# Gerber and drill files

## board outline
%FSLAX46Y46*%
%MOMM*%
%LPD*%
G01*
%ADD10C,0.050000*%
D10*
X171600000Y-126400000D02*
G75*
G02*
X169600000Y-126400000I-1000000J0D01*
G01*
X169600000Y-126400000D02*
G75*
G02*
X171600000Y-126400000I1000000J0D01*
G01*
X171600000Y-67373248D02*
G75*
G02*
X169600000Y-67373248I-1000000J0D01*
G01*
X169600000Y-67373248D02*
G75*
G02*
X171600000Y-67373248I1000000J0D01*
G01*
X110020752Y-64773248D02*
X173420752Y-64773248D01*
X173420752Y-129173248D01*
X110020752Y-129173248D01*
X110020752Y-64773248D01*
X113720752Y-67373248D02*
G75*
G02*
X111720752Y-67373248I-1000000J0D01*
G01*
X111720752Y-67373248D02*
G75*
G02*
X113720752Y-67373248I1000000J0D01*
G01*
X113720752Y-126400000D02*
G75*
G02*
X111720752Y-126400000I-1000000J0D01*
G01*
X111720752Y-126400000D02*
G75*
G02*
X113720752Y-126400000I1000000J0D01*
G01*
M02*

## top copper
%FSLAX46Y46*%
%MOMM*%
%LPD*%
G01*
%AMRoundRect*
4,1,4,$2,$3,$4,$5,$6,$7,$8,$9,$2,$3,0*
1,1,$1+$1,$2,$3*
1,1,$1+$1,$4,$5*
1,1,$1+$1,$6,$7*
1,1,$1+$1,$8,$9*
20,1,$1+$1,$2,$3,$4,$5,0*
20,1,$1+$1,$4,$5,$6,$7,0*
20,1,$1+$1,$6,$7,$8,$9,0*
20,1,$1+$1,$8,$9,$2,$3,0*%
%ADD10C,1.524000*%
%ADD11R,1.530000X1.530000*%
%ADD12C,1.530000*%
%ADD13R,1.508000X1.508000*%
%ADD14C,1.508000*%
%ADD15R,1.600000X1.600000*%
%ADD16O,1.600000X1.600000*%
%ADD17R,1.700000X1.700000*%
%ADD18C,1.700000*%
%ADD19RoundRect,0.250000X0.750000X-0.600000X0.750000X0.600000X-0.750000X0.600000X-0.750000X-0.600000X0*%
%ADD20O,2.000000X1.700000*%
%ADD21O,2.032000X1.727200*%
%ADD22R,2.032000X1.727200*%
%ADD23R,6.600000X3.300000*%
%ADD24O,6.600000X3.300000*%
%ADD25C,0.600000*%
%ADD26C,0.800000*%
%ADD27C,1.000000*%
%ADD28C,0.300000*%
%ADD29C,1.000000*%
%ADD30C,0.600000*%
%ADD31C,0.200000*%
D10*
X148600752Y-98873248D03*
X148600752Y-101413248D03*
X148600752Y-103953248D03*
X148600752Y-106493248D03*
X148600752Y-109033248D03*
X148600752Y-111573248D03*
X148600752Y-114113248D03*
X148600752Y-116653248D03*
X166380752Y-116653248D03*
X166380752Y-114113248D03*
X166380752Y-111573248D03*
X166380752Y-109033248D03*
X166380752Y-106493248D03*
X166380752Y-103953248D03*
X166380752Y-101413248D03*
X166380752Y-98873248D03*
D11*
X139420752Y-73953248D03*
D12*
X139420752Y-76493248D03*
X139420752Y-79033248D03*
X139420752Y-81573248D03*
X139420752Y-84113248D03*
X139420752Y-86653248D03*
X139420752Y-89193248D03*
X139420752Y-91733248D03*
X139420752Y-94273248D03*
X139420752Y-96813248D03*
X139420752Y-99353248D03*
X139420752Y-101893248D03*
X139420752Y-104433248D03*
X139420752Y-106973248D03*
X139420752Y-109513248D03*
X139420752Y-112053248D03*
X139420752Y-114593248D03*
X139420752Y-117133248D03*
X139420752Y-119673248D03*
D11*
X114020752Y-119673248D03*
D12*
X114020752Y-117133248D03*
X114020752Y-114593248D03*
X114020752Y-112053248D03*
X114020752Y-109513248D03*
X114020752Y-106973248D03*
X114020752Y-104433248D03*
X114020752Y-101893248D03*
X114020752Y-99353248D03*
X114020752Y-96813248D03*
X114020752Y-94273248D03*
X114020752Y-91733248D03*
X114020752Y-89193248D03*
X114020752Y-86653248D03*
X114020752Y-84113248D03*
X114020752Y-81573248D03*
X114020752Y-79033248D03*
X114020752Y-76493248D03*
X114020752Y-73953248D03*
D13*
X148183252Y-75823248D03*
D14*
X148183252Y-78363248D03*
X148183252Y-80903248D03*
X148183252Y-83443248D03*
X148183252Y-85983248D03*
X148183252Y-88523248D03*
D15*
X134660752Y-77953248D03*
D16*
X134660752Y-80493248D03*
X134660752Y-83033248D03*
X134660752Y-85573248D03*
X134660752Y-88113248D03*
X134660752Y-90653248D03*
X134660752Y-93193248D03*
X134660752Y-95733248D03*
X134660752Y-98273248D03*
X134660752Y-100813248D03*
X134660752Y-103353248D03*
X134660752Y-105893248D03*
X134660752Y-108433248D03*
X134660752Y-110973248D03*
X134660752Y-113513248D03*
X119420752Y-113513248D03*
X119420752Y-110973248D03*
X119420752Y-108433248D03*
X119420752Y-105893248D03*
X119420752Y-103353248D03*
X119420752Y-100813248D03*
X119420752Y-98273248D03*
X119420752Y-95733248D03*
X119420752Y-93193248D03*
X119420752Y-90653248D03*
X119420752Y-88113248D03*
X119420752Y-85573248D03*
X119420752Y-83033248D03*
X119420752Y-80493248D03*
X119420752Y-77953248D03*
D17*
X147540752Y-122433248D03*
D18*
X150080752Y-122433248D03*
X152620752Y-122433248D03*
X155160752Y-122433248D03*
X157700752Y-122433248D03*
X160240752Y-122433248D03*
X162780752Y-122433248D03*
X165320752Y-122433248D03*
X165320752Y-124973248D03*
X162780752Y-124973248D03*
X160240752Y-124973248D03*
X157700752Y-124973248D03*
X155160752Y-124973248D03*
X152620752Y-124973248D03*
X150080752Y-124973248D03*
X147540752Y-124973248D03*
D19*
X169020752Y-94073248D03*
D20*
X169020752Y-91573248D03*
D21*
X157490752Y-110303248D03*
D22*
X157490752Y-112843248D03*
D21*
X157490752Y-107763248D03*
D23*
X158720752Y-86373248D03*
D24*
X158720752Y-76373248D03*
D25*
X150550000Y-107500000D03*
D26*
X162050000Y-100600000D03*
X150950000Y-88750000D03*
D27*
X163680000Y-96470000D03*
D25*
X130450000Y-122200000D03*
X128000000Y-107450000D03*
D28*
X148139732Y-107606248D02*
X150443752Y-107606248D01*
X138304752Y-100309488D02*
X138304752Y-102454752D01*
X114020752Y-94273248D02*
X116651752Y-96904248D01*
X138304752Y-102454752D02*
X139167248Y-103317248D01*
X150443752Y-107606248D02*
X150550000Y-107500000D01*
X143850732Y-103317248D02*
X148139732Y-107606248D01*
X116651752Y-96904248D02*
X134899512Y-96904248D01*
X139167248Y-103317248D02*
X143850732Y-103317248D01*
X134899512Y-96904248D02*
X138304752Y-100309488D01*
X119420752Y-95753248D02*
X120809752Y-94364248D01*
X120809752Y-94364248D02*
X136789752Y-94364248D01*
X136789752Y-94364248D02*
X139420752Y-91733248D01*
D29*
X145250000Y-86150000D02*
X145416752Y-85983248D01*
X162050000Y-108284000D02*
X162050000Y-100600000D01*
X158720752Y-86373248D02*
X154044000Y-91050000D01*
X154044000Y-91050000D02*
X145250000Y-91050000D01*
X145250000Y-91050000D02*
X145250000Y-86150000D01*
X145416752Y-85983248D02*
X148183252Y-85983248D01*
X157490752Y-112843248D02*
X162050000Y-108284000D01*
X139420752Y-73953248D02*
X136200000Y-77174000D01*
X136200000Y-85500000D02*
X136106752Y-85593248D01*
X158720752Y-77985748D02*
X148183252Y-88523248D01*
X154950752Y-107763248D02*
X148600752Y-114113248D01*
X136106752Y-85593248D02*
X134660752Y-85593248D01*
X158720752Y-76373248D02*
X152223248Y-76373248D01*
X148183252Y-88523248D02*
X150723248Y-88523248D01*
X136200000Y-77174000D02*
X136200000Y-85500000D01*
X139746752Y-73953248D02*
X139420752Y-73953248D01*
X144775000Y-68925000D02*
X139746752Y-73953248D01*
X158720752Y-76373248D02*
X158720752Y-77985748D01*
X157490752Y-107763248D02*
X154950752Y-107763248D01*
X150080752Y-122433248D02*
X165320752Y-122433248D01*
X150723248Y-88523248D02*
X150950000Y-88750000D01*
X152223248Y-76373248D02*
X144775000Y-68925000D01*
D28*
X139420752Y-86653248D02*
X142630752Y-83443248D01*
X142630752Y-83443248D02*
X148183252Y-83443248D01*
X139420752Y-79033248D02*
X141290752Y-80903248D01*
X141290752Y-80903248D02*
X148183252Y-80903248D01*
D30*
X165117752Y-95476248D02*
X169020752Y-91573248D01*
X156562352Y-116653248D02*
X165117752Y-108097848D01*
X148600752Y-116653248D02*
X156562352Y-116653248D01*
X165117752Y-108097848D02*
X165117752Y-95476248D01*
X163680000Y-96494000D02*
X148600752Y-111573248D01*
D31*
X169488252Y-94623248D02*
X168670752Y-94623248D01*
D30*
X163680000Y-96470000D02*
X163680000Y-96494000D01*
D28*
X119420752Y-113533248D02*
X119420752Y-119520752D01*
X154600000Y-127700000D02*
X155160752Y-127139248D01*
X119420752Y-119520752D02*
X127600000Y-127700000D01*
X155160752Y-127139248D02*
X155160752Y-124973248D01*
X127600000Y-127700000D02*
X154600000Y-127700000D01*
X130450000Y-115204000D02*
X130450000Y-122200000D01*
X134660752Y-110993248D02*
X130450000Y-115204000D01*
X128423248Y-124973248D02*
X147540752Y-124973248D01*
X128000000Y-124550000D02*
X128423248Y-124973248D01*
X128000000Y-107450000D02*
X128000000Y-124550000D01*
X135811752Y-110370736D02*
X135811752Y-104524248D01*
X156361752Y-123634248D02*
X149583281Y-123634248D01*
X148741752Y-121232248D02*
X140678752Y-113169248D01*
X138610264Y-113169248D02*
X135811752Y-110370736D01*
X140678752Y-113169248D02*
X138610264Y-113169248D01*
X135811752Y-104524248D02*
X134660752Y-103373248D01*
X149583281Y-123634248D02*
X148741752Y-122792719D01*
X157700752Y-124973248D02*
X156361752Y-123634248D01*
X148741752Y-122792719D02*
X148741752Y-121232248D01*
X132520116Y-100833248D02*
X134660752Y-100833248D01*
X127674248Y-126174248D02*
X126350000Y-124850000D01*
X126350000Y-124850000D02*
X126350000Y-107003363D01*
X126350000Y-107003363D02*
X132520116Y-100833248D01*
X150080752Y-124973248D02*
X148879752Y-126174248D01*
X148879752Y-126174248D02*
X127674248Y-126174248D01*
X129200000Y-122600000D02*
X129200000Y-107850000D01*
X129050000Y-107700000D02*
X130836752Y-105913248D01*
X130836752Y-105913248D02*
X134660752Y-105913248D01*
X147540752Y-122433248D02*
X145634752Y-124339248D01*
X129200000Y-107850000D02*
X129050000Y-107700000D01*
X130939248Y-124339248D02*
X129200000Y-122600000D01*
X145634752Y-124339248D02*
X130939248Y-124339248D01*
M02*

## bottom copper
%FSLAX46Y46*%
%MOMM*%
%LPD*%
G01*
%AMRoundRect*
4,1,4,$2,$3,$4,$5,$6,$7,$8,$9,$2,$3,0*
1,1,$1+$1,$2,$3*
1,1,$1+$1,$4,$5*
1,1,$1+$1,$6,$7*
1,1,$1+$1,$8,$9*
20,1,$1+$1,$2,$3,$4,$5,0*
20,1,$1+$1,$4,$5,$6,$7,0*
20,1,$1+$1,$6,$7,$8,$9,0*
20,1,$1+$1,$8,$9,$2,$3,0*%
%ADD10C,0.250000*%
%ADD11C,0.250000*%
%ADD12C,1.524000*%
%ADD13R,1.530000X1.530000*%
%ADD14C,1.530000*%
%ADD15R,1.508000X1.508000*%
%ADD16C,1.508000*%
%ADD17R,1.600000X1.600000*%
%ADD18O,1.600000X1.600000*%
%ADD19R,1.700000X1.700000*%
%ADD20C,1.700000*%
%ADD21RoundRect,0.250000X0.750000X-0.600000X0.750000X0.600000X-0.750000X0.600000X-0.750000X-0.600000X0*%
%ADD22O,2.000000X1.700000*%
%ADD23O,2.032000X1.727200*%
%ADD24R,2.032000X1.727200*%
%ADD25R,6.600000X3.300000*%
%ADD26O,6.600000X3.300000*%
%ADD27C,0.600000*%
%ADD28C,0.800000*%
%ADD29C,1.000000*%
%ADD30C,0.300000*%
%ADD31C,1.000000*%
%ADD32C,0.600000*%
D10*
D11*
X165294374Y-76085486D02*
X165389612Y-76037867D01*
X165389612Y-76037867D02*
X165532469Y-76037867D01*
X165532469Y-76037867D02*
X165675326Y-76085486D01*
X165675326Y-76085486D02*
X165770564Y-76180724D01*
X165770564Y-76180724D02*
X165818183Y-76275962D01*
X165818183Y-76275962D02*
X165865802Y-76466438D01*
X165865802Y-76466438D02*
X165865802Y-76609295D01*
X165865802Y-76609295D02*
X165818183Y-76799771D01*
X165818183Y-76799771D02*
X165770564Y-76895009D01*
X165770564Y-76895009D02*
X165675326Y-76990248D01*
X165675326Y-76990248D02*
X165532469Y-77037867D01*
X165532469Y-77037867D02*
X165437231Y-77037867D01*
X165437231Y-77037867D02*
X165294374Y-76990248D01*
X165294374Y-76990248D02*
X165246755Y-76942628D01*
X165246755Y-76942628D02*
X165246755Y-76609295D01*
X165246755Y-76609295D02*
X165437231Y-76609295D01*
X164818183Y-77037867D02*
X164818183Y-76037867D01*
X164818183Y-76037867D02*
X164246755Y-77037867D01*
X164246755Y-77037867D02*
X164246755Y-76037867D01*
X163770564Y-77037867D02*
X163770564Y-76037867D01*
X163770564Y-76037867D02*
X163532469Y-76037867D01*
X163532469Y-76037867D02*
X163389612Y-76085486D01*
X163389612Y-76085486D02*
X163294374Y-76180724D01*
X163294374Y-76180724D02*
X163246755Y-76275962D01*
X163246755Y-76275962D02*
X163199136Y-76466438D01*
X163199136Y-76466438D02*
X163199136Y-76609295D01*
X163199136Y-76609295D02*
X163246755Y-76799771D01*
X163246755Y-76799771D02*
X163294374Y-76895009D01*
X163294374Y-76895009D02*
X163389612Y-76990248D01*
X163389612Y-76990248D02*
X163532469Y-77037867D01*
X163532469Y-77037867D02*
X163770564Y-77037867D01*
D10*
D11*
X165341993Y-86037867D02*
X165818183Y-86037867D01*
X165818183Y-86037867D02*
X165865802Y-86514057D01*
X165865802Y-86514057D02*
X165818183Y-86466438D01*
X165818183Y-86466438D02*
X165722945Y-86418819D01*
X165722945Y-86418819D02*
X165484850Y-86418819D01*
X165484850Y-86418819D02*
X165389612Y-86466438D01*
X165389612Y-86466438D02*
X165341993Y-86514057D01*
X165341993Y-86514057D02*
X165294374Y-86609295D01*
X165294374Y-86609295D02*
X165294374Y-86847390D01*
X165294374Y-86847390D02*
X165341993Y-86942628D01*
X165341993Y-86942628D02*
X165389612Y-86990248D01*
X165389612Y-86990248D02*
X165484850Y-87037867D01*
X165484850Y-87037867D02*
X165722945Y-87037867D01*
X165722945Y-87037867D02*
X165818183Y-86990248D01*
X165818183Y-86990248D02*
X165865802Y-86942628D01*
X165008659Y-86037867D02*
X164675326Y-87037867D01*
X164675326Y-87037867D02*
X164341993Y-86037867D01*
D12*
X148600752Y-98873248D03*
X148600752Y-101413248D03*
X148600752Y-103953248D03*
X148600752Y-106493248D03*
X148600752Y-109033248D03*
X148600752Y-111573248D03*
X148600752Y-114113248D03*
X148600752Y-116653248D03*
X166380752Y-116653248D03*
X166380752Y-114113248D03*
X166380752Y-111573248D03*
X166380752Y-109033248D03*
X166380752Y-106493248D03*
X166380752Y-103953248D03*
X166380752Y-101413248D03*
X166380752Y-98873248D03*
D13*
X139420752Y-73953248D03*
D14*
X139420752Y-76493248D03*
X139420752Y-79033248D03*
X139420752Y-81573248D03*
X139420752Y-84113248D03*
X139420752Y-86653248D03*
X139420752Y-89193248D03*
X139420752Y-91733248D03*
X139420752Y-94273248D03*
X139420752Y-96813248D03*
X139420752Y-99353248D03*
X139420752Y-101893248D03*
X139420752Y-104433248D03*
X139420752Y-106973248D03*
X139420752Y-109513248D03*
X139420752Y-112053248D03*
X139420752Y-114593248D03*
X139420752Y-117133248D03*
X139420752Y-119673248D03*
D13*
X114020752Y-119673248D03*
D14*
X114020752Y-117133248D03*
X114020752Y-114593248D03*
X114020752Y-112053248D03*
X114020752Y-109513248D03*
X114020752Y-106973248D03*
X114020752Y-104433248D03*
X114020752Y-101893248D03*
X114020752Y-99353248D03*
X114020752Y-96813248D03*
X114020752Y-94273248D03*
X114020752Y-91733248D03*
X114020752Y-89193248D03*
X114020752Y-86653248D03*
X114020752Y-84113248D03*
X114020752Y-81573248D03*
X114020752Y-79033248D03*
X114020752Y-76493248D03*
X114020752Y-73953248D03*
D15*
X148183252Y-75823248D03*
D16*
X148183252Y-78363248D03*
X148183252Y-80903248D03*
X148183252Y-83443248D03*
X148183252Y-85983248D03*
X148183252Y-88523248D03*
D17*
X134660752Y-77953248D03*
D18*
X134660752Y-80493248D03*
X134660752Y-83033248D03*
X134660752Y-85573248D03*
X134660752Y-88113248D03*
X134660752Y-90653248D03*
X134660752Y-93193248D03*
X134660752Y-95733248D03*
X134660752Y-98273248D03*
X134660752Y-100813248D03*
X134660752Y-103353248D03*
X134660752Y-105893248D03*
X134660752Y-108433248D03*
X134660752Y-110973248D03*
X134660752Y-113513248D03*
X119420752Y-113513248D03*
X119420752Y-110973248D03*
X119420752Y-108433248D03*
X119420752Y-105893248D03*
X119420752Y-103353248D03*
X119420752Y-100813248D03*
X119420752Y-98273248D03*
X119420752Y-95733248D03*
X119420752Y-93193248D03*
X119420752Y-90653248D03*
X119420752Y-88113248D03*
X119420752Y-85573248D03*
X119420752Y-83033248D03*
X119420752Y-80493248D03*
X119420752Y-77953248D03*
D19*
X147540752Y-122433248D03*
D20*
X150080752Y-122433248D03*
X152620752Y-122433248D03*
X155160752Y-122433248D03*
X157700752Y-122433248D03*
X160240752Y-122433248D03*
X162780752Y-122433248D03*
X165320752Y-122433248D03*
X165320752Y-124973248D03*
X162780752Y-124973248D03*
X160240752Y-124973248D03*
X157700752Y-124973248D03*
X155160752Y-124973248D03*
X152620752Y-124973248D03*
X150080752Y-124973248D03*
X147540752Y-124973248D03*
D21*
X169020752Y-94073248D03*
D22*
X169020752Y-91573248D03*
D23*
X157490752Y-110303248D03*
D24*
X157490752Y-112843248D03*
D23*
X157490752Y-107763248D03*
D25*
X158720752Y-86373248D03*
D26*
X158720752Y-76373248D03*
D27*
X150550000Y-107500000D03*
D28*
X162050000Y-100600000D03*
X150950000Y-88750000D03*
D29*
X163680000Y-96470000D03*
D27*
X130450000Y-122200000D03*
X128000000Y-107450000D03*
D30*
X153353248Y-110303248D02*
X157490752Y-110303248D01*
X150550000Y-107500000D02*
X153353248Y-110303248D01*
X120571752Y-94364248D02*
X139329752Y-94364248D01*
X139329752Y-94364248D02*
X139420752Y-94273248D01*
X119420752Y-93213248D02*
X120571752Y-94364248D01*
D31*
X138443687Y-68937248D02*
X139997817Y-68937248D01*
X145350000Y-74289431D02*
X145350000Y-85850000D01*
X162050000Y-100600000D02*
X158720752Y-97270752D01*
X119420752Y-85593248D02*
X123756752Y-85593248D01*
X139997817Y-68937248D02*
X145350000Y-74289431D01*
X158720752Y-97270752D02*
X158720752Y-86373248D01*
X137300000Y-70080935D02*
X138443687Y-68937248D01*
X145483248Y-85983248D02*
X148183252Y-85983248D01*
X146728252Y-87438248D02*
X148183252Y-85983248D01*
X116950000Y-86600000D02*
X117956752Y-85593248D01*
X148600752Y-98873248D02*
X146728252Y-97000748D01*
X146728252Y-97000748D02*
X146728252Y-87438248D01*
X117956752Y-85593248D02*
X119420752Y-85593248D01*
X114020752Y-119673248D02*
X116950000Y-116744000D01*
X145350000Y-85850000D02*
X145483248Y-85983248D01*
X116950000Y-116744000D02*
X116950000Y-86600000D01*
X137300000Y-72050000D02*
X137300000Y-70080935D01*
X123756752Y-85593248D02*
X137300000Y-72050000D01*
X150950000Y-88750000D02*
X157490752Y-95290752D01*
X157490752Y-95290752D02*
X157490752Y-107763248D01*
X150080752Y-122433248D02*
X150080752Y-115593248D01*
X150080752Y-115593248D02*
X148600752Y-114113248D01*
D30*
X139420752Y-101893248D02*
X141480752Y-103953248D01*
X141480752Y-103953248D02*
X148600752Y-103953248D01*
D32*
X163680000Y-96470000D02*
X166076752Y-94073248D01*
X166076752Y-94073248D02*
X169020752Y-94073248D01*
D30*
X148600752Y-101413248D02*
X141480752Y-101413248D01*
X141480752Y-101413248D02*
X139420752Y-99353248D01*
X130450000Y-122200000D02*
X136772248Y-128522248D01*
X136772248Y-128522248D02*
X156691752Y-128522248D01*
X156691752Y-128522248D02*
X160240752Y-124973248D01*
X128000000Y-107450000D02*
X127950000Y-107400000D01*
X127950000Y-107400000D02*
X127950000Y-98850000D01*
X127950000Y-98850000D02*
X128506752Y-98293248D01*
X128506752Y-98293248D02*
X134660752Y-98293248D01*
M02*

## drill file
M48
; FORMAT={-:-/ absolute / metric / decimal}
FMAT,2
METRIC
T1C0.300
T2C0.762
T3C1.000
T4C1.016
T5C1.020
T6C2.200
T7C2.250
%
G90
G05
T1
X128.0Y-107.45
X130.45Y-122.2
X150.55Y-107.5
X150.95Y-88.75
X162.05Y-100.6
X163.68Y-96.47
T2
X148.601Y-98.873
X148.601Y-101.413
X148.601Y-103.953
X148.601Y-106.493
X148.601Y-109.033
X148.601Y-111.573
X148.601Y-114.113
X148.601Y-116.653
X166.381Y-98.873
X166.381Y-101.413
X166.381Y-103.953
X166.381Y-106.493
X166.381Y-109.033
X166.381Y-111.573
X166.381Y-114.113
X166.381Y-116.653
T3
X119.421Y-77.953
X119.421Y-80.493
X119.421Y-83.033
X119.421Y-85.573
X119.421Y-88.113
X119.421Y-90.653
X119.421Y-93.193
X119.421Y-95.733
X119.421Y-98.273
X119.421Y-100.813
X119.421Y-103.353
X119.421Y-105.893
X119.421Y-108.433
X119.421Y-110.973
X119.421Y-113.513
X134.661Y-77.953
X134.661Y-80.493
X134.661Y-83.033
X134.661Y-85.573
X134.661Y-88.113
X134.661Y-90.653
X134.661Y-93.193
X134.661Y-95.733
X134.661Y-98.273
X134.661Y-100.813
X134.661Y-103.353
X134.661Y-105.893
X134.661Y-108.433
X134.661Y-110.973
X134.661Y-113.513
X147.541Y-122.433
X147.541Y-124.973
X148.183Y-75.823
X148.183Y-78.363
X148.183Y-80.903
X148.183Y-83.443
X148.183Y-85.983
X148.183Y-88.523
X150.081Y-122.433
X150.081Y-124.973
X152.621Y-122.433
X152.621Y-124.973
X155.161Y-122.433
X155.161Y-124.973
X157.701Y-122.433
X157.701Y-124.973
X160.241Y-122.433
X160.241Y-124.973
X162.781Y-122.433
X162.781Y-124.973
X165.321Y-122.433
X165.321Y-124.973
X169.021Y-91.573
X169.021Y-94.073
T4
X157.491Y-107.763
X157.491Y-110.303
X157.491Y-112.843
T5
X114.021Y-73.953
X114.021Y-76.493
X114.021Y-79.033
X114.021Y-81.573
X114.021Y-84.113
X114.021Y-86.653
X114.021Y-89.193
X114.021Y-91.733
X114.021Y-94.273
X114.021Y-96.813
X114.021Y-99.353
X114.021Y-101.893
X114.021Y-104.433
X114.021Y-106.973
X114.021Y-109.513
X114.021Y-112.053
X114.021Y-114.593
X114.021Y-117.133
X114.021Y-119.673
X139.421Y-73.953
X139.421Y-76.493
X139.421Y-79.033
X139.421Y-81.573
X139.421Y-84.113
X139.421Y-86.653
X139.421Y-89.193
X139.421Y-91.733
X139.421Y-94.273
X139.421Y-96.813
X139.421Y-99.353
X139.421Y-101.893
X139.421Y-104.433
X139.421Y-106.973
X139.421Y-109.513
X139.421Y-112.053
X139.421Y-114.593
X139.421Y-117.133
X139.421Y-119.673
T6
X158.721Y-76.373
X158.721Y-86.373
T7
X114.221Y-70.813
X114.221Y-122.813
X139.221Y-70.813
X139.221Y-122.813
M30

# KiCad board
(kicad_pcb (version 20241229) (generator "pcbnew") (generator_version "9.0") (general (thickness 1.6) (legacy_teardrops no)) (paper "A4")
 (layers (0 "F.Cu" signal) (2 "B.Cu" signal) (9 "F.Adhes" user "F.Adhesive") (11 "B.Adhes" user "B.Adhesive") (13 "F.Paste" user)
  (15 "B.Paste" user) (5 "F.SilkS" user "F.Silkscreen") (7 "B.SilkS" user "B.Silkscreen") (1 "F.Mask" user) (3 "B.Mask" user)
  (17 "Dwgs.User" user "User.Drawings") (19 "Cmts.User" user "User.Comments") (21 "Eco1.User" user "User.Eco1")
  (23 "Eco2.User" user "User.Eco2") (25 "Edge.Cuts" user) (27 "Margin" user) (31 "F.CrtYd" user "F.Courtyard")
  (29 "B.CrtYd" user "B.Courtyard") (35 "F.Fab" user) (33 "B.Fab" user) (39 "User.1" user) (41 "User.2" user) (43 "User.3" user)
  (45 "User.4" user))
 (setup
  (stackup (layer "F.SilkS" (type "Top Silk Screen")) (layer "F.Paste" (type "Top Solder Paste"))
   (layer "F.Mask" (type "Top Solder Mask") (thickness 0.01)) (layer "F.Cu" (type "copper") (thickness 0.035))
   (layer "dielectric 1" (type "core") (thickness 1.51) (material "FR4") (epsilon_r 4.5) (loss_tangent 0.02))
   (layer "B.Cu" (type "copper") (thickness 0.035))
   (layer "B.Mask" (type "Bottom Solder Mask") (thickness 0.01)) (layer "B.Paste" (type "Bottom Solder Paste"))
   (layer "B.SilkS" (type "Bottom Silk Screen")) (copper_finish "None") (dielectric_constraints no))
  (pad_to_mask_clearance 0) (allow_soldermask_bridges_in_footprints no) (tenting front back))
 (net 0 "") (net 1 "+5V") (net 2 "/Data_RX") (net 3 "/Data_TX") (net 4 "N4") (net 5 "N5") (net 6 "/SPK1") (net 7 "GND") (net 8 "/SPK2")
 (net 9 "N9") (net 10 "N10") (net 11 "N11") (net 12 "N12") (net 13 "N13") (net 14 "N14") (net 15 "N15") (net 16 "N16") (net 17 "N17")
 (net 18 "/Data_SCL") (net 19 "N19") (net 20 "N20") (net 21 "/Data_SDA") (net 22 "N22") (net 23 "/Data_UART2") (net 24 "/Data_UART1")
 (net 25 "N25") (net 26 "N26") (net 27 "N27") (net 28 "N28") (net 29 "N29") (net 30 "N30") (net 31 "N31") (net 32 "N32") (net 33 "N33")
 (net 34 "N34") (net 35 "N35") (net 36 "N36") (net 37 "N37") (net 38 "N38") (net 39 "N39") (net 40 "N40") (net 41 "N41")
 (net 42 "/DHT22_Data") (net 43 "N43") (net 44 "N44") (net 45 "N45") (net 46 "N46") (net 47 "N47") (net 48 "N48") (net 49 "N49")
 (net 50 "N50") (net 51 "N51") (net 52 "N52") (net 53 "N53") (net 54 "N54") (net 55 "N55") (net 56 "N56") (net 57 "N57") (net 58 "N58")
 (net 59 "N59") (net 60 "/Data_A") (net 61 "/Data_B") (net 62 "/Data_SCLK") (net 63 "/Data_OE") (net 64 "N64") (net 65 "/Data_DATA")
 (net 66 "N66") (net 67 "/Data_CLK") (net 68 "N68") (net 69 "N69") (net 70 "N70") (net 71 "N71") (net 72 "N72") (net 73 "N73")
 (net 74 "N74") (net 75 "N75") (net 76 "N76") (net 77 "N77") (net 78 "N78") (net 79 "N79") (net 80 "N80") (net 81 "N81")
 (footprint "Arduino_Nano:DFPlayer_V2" (layer "F.Cu") (at 156.220752 98.873248)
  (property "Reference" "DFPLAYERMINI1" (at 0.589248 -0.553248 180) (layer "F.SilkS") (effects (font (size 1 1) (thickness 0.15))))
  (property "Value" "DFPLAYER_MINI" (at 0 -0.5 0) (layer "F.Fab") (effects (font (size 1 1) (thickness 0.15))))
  (pad "1" thru_hole circle (at -7.62 0) (size 1.524 1.524) (drill 0.762) (layers "*.Cu" "*.Mask") (remove_unused_layers no) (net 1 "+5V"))
  (pad "2" thru_hole circle (at -7.62 2.54) (size 1.524 1.524) (drill 0.762) (layers "*.Cu" "*.Mask") (remove_unused_layers no)
   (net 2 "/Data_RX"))
  (pad "3" thru_hole circle (at -7.62 5.08) (size 1.524 1.524) (drill 0.762) (layers "*.Cu" "*.Mask") (remove_unused_layers no)
   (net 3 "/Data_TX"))
  (pad "4" thru_hole circle (at -7.62 7.62) (size 1.524 1.524) (drill 0.762) (layers "*.Cu" "*.Mask") (remove_unused_layers no) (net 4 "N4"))
  (pad "5" thru_hole circle (at -7.62 10.16) (size 1.524 1.524) (drill 0.762) (layers "*.Cu" "*.Mask") (remove_unused_layers no)
   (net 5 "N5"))
  (pad "6" thru_hole circle (at -7.62 12.7) (size 1.524 1.524) (drill 0.762) (layers "*.Cu" "*.Mask") (remove_unused_layers no)
   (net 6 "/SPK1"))
  (pad "7" thru_hole circle (at -7.62 15.24) (size 1.524 1.524) (drill 0.762) (layers "*.Cu" "*.Mask") (remove_unused_layers no)
   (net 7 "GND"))
  (pad "8" thru_hole circle (at -7.62 17.78) (size 1.524 1.524) (drill 0.762) (layers "*.Cu" "*.Mask") (remove_unused_layers no)
   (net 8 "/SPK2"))
  (pad "9" thru_hole circle (at 10.16 17.78) (size 1.524 1.524) (drill 0.762) (layers "*.Cu" "*.Mask") (remove_unused_layers no)
   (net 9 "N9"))
  (pad "10" thru_hole circle (at 10.16 15.24) (size 1.524 1.524) (drill 0.762) (layers "*.Cu" "*.Mask") (remove_unused_layers no)
   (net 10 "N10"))
  (pad "11" thru_hole circle (at 10.16 12.7) (size 1.524 1.524) (drill 0.762) (layers "*.Cu" "*.Mask") (remove_unused_layers no)
   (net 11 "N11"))
  (pad "12" thru_hole circle (at 10.16 10.16) (size 1.524 1.524) (drill 0.762) (layers "*.Cu" "*.Mask") (remove_unused_layers no)
   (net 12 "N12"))
  (pad "13" thru_hole circle (at 10.16 7.62) (size 1.524 1.524) (drill 0.762) (layers "*.Cu" "*.Mask") (remove_unused_layers no)
   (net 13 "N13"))
  (pad "14" thru_hole circle (at 10.16 5.08) (size 1.524 1.524) (drill 0.762) (layers "*.Cu" "*.Mask") (remove_unused_layers no)
   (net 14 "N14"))
  (pad "15" thru_hole circle (at 10.16 2.54) (size 1.524 1.524) (drill 0.762) (layers "*.Cu" "*.Mask") (remove_unused_layers no)
   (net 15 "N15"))
  (pad "16" thru_hole circle (at 10.16 0) (size 1.524 1.524) (drill 0.762) (layers "*.Cu" "*.Mask") (remove_unused_layers no) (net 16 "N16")))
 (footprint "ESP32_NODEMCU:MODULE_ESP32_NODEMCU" (layer "F.Cu") (at 126.720752 96.813248)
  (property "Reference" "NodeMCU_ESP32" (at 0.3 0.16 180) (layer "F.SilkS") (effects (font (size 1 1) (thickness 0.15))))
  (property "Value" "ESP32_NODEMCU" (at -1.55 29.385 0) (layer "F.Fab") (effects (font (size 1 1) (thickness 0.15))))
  (pad "" np_thru_hole circle (at -12.5 -26) (size 2.25 2.25) (drill 2.25) (layers "*.Cu" "*.Mask"))
  (pad "" np_thru_hole circle (at -12.5 26) (size 2.25 2.25) (drill 2.25) (layers "*.Cu" "*.Mask"))
  (pad "" np_thru_hole circle (at 12.5 -26) (size 2.25 2.25) (drill 2.25) (layers "*.Cu" "*.Mask"))
  (pad "" np_thru_hole circle (at 12.5 26) (size 2.25 2.25) (drill 2.25) (layers "*.Cu" "*.Mask"))
  (pad "J4_1" thru_hole rect (at 12.7 -22.86) (size 1.53 1.53) (drill 1.02) (layers "*.Cu" "*.Mask") (remove_unused_layers no) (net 7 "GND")
   (solder_mask_margin 0.102))
  (pad "J4_2" thru_hole circle (at 12.7 -20.32) (size 1.53 1.53) (drill 1.02) (layers "*.Cu" "*.Mask") (remove_unused_layers no)
   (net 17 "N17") (solder_mask_margin 0.102))
  (pad "J4_3" thru_hole circle (at 12.7 -17.78) (size 1.53 1.53) (drill 1.02) (layers "*.Cu" "*.Mask") (remove_unused_layers no)
   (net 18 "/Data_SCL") (solder_mask_margin 0.102))
  (pad "J4_4" thru_hole circle (at 12.7 -15.24) (size 1.53 1.53) (drill 1.02) (layers "*.Cu" "*.Mask") (remove_unused_layers no)
   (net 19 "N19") (solder_mask_margin 0.102))
  (pad "J4_5" thru_hole circle (at 12.7 -12.7) (size 1.53 1.53) (drill 1.02) (layers "*.Cu" "*.Mask") (remove_unused_layers no)
   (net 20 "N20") (solder_mask_margin 0.102))
  (pad "J4_6" thru_hole circle (at 12.7 -10.16) (size 1.53 1.53) (drill 1.02) (layers "*.Cu" "*.Mask") (remove_unused_layers no)
   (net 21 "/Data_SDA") (solder_mask_margin 0.102))
  (pad "J4_7" thru_hole circle (at 12.7 -7.62) (size 1.53 1.53) (drill 1.02) (layers "*.Cu" "*.Mask") (remove_unused_layers no)
   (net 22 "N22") (solder_mask_margin 0.102))
  (pad "J4_8" thru_hole circle (at 12.7 -5.08) (size 1.53 1.53) (drill 1.02) (layers "*.Cu" "*.Mask") (remove_unused_layers no)
   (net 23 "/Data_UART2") (solder_mask_margin 0.102))
  (pad "J4_9" thru_hole circle (at 12.7 -2.54) (size 1.53 1.53) (drill 1.02) (layers "*.Cu" "*.Mask") (remove_unused_layers no)
   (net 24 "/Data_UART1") (solder_mask_margin 0.102))
  (pad "J4_10" thru_hole circle (at 12.7 0) (size 1.53 1.53) (drill 1.02) (layers "*.Cu" "*.Mask") (remove_unused_layers no) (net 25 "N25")
   (solder_mask_margin 0.102))
  (pad "J4_11" thru_hole circle (at 12.7 2.54) (size 1.53 1.53) (drill 1.02) (layers "*.Cu" "*.Mask") (remove_unused_layers no)
   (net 2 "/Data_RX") (solder_mask_margin 0.102))
  (pad "J4_12" thru_hole circle (at 12.7 5.08) (size 1.53 1.53) (drill 1.02) (layers "*.Cu" "*.Mask") (remove_unused_layers no)
   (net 3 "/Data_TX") (solder_mask_margin 0.102))
  (pad "J4_13" thru_hole circle (at 12.7 7.62) (size 1.53 1.53) (drill 1.02) (layers "*.Cu" "*.Mask") (remove_unused_layers no)
   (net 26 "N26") (solder_mask_margin 0.102))
  (pad "J4_14" thru_hole circle (at 12.7 10.16) (size 1.53 1.53) (drill 1.02) (layers "*.Cu" "*.Mask") (remove_unused_layers no)
   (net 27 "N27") (solder_mask_margin 0.102))
  (pad "J4_15" thru_hole circle (at 12.7 12.7) (size 1.53 1.53) (drill 1.02) (layers "*.Cu" "*.Mask") (remove_unused_layers no)
   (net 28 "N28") (solder_mask_margin 0.102))
  (pad "J4_16" thru_hole circle (at 12.7 15.24) (size 1.53 1.53) (drill 1.02) (layers "*.Cu" "*.Mask") (remove_unused_layers no)
   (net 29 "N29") (solder_mask_margin 0.102))
  (pad "J4_17" thru_hole circle (at 12.7 17.78) (size 1.53 1.53) (drill 1.02) (layers "*.Cu" "*.Mask") (remove_unused_layers no)
   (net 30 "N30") (solder_mask_margin 0.102))
  (pad "J4_18" thru_hole circle (at 12.7 20.32) (size 1.53 1.53) (drill 1.02) (layers "*.Cu" "*.Mask") (remove_unused_layers no)
   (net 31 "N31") (solder_mask_margin 0.102))
  (pad "J4_19" thru_hole circle (at 12.7 22.86) (size 1.53 1.53) (drill 1.02) (layers "*.Cu" "*.Mask") (remove_unused_layers no)
   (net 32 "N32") (solder_mask_margin 0.102))
  (pad "J5_1" thru_hole rect (at -12.7 22.86) (size 1.53 1.53) (drill 1.02) (layers "*.Cu" "*.Mask") (remove_unused_layers no) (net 1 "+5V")
   (solder_mask_margin 0.102))
  (pad "J5_2" thru_hole circle (at -12.7 20.32) (size 1.53 1.53) (drill 1.02) (layers "*.Cu" "*.Mask") (remove_unused_layers no)
   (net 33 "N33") (solder_mask_margin 0.102))
  (pad "J5_3" thru_hole circle (at -12.7 17.78) (size 1.53 1.53) (drill 1.02) (layers "*.Cu" "*.Mask") (remove_unused_layers no)
   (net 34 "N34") (solder_mask_margin 0.102))
  (pad "J5_4" thru_hole circle (at -12.7 15.24) (size 1.53 1.53) (drill 1.02) (layers "*.Cu" "*.Mask") (remove_unused_layers no)
   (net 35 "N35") (solder_mask_margin 0.102))
  (pad "J5_5" thru_hole circle (at -12.7 12.7) (size 1.53 1.53) (drill 1.02) (layers "*.Cu" "*.Mask") (remove_unused_layers no)
   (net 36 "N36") (solder_mask_margin 0.102))
  (pad "J5_6" thru_hole circle (at -12.7 10.16) (size 1.53 1.53) (drill 1.02) (layers "*.Cu" "*.Mask") (remove_unused_layers no)
   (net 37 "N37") (solder_mask_margin 0.102))
  (pad "J5_7" thru_hole circle (at -12.7 7.62) (size 1.53 1.53) (drill 1.02) (layers "*.Cu" "*.Mask") (remove_unused_layers no)
   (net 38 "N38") (solder_mask_margin 0.102))
  (pad "J5_8" thru_hole circle (at -12.7 5.08) (size 1.53 1.53) (drill 1.02) (layers "*.Cu" "*.Mask") (remove_unused_layers no)
   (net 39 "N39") (solder_mask_margin 0.102))
  (pad "J5_9" thru_hole circle (at -12.7 2.54) (size 1.53 1.53) (drill 1.02) (layers "*.Cu" "*.Mask") (remove_unused_layers no)
   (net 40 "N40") (solder_mask_margin 0.102))
  (pad "J5_10" thru_hole circle (at -12.7 0) (size 1.53 1.53) (drill 1.02) (layers "*.Cu" "*.Mask") (remove_unused_layers no) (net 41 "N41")
   (solder_mask_margin 0.102))
  (pad "J5_11" thru_hole circle (at -12.7 -2.54) (size 1.53 1.53) (drill 1.02) (layers "*.Cu" "*.Mask") (remove_unused_layers no)
   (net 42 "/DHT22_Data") (solder_mask_margin 0.102))
  (pad "J5_12" thru_hole circle (at -12.7 -5.08) (size 1.53 1.53) (drill 1.02) (layers "*.Cu" "*.Mask") (remove_unused_layers no)
   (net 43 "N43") (solder_mask_margin 0.102))
  (pad "J5_13" thru_hole circle (at -12.7 -7.62) (size 1.53 1.53) (drill 1.02) (layers "*.Cu" "*.Mask") (remove_unused_layers no)
   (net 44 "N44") (solder_mask_margin 0.102))
  (pad "J5_14" thru_hole circle (at -12.7 -10.16) (size 1.53 1.53) (drill 1.02) (layers "*.Cu" "*.Mask") (remove_unused_layers no)
   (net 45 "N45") (solder_mask_margin 0.102))
  (pad "J5_15" thru_hole circle (at -12.7 -12.7) (size 1.53 1.53) (drill 1.02) (layers "*.Cu" "*.Mask") (remove_unused_layers no)
   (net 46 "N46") (solder_mask_margin 0.102))
  (pad "J5_16" thru_hole circle (at -12.7 -15.24) (size 1.53 1.53) (drill 1.02) (layers "*.Cu" "*.Mask") (remove_unused_layers no)
   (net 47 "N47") (solder_mask_margin 0.102))
  (pad "J5_17" thru_hole circle (at -12.7 -17.78) (size 1.53 1.53) (drill 1.02) (layers "*.Cu" "*.Mask") (remove_unused_layers no)
   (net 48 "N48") (solder_mask_margin 0.102))
  (pad "J5_18" thru_hole circle (at -12.7 -20.32) (size 1.53 1.53) (drill 1.02) (layers "*.Cu" "*.Mask") (remove_unused_layers no)
   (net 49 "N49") (solder_mask_margin 0.102))
  (pad "J5_19" thru_hole circle (at -12.7 -22.86) (size 1.53 1.53) (drill 1.02) (layers "*.Cu" "*.Mask") (remove_unused_layers no)
   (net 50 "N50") (solder_mask_margin 0.102)))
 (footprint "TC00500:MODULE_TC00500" (layer "F.Cu") (at 148.183252 82.173248)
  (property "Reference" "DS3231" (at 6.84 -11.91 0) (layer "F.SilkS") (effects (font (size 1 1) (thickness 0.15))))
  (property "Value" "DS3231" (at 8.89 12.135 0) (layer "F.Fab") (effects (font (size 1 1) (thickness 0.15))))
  (pad "1" thru_hole rect (at 0 -6.35) (size 1.508 1.508) (drill 1) (layers "*.Cu" "*.Mask") (remove_unused_layers no) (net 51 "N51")
   (solder_mask_margin 0.102))
  (pad "2" thru_hole circle (at 0 -3.81) (size 1.508 1.508) (drill 1) (layers "*.Cu" "*.Mask") (remove_unused_layers no) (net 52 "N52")
   (solder_mask_margin 0.102))
  (pad "3" thru_hole circle (at 0 -1.27) (size 1.508 1.508) (drill 1) (layers "*.Cu" "*.Mask") (remove_unused_layers no)
   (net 18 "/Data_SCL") (solder_mask_margin 0.102))
  (pad "4" thru_hole circle (at 0 1.27) (size 1.508 1.508) (drill 1) (layers "*.Cu" "*.Mask") (remove_unused_layers no) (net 21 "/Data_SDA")
   (solder_mask_margin 0.102))
  (pad "5" thru_hole circle (at 0 3.81) (size 1.508 1.508) (drill 1) (layers "*.Cu" "*.Mask") (remove_unused_layers no) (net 1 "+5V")
   (solder_mask_margin 0.102))
  (pad "6" thru_hole circle (at 0 6.35) (size 1.508 1.508) (drill 1) (layers "*.Cu" "*.Mask") (remove_unused_layers no) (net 7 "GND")
   (solder_mask_margin 0.102)))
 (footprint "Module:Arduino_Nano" (layer "B.Cu") (at 134.660752 77.953248 180)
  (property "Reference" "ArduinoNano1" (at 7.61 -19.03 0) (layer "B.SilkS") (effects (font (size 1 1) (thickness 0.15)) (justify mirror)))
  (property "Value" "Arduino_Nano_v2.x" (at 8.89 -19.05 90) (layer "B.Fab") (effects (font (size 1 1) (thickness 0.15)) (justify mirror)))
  (pad "1" thru_hole rect (at 0 0 180) (size 1.6 1.6) (drill 1) (layers "*.Cu" "*.Mask") (remove_unused_layers no) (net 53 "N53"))
  (pad "2" thru_hole oval (at 0 -2.54 180) (size 1.6 1.6) (drill 1) (layers "*.Cu" "*.Mask") (remove_unused_layers no) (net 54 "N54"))
  (pad "3" thru_hole oval (at 0 -5.08 180) (size 1.6 1.6) (drill 1) (layers "*.Cu" "*.Mask") (remove_unused_layers no) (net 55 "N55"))
  (pad "4" thru_hole oval (at 0 -7.62 180) (size 1.6 1.6) (drill 1) (layers "*.Cu" "*.Mask") (remove_unused_layers no) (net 7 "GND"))
  (pad "5" thru_hole oval (at 0 -10.16 180) (size 1.6 1.6) (drill 1) (layers "*.Cu" "*.Mask") (remove_unused_layers no) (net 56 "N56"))
  (pad "6" thru_hole oval (at 0 -12.7 180) (size 1.6 1.6) (drill 1) (layers "*.Cu" "*.Mask") (remove_unused_layers no) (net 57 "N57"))
  (pad "7" thru_hole oval (at 0 -15.24 180) (size 1.6 1.6) (drill 1) (layers "*.Cu" "*.Mask") (remove_unused_layers no) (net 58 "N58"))
  (pad "8" thru_hole oval (at 0 -17.78 180) (size 1.6 1.6) (drill 1) (layers "*.Cu" "*.Mask") (remove_unused_layers no) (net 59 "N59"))
  (pad "9" thru_hole oval (at 0 -20.32 180) (size 1.6 1.6) (drill 1) (layers "*.Cu" "*.Mask") (remove_unused_layers no) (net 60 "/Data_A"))
  (pad "10" thru_hole oval (at 0 -22.86 180) (size 1.6 1.6) (drill 1) (layers "*.Cu" "*.Mask") (remove_unused_layers no) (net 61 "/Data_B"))
  (pad "11" thru_hole oval (at 0 -25.4 180) (size 1.6 1.6) (drill 1) (layers "*.Cu" "*.Mask") (remove_unused_layers no)
   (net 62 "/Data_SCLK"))
  (pad "12" thru_hole oval (at 0 -27.94 180) (size 1.6 1.6) (drill 1) (layers "*.Cu" "*.Mask") (remove_unused_layers no) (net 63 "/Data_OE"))
  (pad "13" thru_hole oval (at 0 -30.48 180) (size 1.6 1.6) (drill 1) (layers "*.Cu" "*.Mask") (remove_unused_layers no) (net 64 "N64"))
  (pad "14" thru_hole oval (at 0 -33.02 180) (size 1.6 1.6) (drill 1) (layers "*.Cu" "*.Mask") (remove_unused_layers no)
   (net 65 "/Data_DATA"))
  (pad "15" thru_hole oval (at 0 -35.56 180) (size 1.6 1.6) (drill 1) (layers "*.Cu" "*.Mask") (remove_unused_layers no) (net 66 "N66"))
  (pad "16" thru_hole oval (at 15.24 -35.56 180) (size 1.6 1.6) (drill 1) (layers "*.Cu" "*.Mask") (remove_unused_layers no)
   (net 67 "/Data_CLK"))
  (pad "17" thru_hole oval (at 15.24 -33.02 180) (size 1.6 1.6) (drill 1) (layers "*.Cu" "*.Mask") (remove_unused_layers no) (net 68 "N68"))
  (pad "18" thru_hole oval (at 15.24 -30.48 180) (size 1.6 1.6) (drill 1) (layers "*.Cu" "*.Mask") (remove_unused_layers no) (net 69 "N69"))
  (pad "19" thru_hole oval (at 15.24 -27.94 180) (size 1.6 1.6) (drill 1) (layers "*.Cu" "*.Mask") (remove_unused_layers no) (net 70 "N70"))
  (pad "20" thru_hole oval (at 15.24 -25.4 180) (size 1.6 1.6) (drill 1) (layers "*.Cu" "*.Mask") (remove_unused_layers no) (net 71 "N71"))
  (pad "21" thru_hole oval (at 15.24 -22.86 180) (size 1.6 1.6) (drill 1) (layers "*.Cu" "*.Mask") (remove_unused_layers no) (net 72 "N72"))
  (pad "22" thru_hole oval (at 15.24 -20.32 180) (size 1.6 1.6) (drill 1) (layers "*.Cu" "*.Mask") (remove_unused_layers no) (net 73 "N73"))
  (pad "23" thru_hole oval (at 15.24 -17.78 180) (size 1.6 1.6) (drill 1) (layers "*.Cu" "*.Mask") (remove_unused_layers no)
   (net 23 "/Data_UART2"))
  (pad "24" thru_hole oval (at 15.24 -15.24 180) (size 1.6 1.6) (drill 1) (layers "*.Cu" "*.Mask") (remove_unused_layers no)
   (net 24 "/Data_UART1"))
  (pad "25" thru_hole oval (at 15.24 -12.7 180) (size 1.6 1.6) (drill 1) (layers "*.Cu" "*.Mask") (remove_unused_layers no) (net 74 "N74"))
  (pad "26" thru_hole oval (at 15.24 -10.16 180) (size 1.6 1.6) (drill 1) (layers "*.Cu" "*.Mask") (remove_unused_layers no) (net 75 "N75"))
  (pad "27" thru_hole oval (at 15.24 -7.62 180) (size 1.6 1.6) (drill 1) (layers "*.Cu" "*.Mask") (remove_unused_layers no) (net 1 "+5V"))
  (pad "28" thru_hole oval (at 15.24 -5.08 180) (size 1.6 1.6) (drill 1) (layers "*.Cu" "*.Mask") (remove_unused_layers no) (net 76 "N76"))
  (pad "29" thru_hole oval (at 15.24 -2.54 180) (size 1.6 1.6) (drill 1) (layers "*.Cu" "*.Mask") (remove_unused_layers no) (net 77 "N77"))
  (pad "30" thru_hole oval (at 15.24 0 180) (size 1.6 1.6) (drill 1) (layers "*.Cu" "*.Mask") (remove_unused_layers no) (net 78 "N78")))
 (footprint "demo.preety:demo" (layer "B.Cu") (at 171.32 101.57 -90)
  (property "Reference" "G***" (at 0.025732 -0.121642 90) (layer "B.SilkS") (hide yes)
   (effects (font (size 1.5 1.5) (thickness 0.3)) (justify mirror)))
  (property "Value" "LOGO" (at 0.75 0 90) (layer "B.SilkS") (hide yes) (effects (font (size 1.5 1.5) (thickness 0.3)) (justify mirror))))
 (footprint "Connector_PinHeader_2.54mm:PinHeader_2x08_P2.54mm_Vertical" (layer "B.Cu") (at 147.540752 122.433248 -90)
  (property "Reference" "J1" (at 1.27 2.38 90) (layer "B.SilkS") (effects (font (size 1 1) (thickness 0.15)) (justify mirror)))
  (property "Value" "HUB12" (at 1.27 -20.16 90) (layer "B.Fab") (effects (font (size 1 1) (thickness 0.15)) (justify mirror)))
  (pad "1" thru_hole rect (at 0 0 270) (size 1.7 1.7) (drill 1) (layers "*.Cu" "*.Mask") (remove_unused_layers no) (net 63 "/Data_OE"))
  (pad "2" thru_hole circle (at 0 -2.54 270) (size 1.7 1.7) (drill 1) (layers "*.Cu" "*.Mask") (remove_unused_layers no) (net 7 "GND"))
  (pad "3" thru_hole circle (at 0 -5.08 270) (size 1.7 1.7) (drill 1) (layers "*.Cu" "*.Mask") (remove_unused_layers no) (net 7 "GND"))
  (pad "4" thru_hole circle (at 0 -7.62 270) (size 1.7 1.7) (drill 1) (layers "*.Cu" "*.Mask") (remove_unused_layers no) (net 7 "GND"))
  (pad "5" thru_hole circle (at 0 -10.16 270) (size 1.7 1.7) (drill 1) (layers "*.Cu" "*.Mask") (remove_unused_layers no) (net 7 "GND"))
  (pad "6" thru_hole circle (at 0 -12.7 270) (size 1.7 1.7) (drill 1) (layers "*.Cu" "*.Mask") (remove_unused_layers no) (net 7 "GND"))
  (pad "7" thru_hole circle (at 0 -15.24 270) (size 1.7 1.7) (drill 1) (layers "*.Cu" "*.Mask") (remove_unused_layers no) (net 7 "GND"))
  (pad "8" thru_hole circle (at 0 -17.78 270) (size 1.7 1.7) (drill 1) (layers "*.Cu" "*.Mask") (remove_unused_layers no) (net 7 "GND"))
  (pad "9" thru_hole circle (at 2.54 -17.78 270) (size 1.7 1.7) (drill 1) (layers "*.Cu" "*.Mask") (remove_unused_layers no) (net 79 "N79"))
  (pad "10" thru_hole circle (at 2.54 -15.24 270) (size 1.7 1.7) (drill 1) (layers "*.Cu" "*.Mask") (remove_unused_layers no) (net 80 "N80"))
  (pad "11" thru_hole circle (at 2.54 -12.7 270) (size 1.7 1.7) (drill 1) (layers "*.Cu" "*.Mask") (remove_unused_layers no)
   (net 65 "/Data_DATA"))
  (pad "12" thru_hole circle (at 2.54 -10.16 270) (size 1.7 1.7) (drill 1) (layers "*.Cu" "*.Mask") (remove_unused_layers no)
   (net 62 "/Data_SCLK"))
  (pad "13" thru_hole circle (at 2.54 -7.62 270) (size 1.7 1.7) (drill 1) (layers "*.Cu" "*.Mask") (remove_unused_layers no)
   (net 67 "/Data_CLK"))
  (pad "14" thru_hole circle (at 2.54 -5.08 270) (size 1.7 1.7) (drill 1) (layers "*.Cu" "*.Mask") (remove_unused_layers no) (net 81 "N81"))
  (pad "15" thru_hole circle (at 2.54 -2.54 270) (size 1.7 1.7) (drill 1) (layers "*.Cu" "*.Mask") (remove_unused_layers no)
   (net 61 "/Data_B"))
  (pad "16" thru_hole circle (at 2.54 0 270) (size 1.7 1.7) (drill 1) (layers "*.Cu" "*.Mask") (remove_unused_layers no) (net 60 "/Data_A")))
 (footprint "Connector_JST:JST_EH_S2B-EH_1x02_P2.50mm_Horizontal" (layer "B.Cu") (at 169.020752 94.073248 90)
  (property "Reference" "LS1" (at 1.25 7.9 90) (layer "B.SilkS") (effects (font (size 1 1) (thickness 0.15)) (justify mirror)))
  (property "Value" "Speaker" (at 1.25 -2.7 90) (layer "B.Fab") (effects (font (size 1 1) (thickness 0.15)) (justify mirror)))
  (pad "1" thru_hole roundrect (at 0 0 90) (size 1.7 2) (drill 1) (layers "*.Cu" "*.Mask") (remove_unused_layers no)
   (roundrect_rratio 0.147059) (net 6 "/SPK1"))
  (pad "2" thru_hole oval (at 2.5 0 90) (size 1.7 2) (drill 1) (layers "*.Cu" "*.Mask") (remove_unused_layers no) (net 8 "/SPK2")))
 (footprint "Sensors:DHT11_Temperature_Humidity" (layer "B.Cu") (at 157.490752 110.303248 -90)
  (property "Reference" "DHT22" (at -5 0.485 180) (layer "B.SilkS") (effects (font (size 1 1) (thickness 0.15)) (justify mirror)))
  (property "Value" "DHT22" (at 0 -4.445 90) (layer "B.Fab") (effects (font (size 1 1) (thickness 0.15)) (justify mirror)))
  (pad "1" thru_hole oval (at 0 0) (size 2.032 1.7272) (drill 1.016) (layers "*.Cu" "F.Mask" "B.SilkS") (remove_unused_layers no)
   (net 42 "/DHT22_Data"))
  (pad "2" thru_hole rect (at 2.54 0) (size 2.032 1.7272) (drill 1.016) (layers "*.Cu" "F.Mask" "B.SilkS") (remove_unused_layers no)
   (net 1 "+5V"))
  (pad "3" thru_hole oval (at -2.54 0) (size 2.032 1.7272) (drill 1.016) (layers "*.Cu" "F.Mask" "B.SilkS") (remove_unused_layers no)
   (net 7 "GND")))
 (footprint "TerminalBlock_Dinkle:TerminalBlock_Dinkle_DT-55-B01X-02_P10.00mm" (layer "B.Cu") (at 158.720752 86.373248 90)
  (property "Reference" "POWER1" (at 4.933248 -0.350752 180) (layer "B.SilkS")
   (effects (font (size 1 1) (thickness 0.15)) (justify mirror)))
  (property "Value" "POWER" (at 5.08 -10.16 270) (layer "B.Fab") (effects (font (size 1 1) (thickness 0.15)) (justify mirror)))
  (pad "1" thru_hole rect (at 0 0 90) (size 3.3 6.6) (drill 2.2) (layers "*.Cu" "*.Mask") (remove_unused_layers no) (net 1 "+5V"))
  (pad "2" thru_hole oval (at 10 0 90) (size 3.3 6.6) (drill 2.2) (layers "*.Cu" "*.Mask") (remove_unused_layers no) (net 7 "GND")))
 (gr_circle (center 170.6 126.4) (end 171.6 126.4) (stroke (width 0.05) (type solid)) (fill no) (layer "Edge.Cuts"))
 (gr_circle (center 170.6 67.373248) (end 171.6 67.373248) (stroke (width 0.05) (type solid)) (fill no) (layer "Edge.Cuts"))
 (gr_rect (start 110.020752 64.773248) (end 173.420752 129.173248) (stroke (width 0.05) (type default)) (fill no) (layer "Edge.Cuts"))
 (gr_circle (center 112.720752 67.373248) (end 113.720752 67.373248) (stroke (width 0.05) (type solid)) (fill no) (layer "Edge.Cuts"))
 (gr_circle (center 112.720752 126.4) (end 113.720752 126.4) (stroke (width 0.05) (type solid)) (fill no) (layer "Edge.Cuts"))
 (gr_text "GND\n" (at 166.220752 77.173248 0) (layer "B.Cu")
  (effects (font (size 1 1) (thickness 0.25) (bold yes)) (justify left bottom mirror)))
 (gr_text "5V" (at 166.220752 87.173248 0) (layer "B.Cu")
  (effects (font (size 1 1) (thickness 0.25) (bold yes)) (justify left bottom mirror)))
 (segment (start 148.139732 107.606248) (end 150.443752 107.606248) (width 0.3) (layer "F.Cu") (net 42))
 (segment (start 138.304752 100.309488) (end 138.304752 102.454752) (width 0.3) (layer "F.Cu") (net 42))
 (segment (start 114.020752 94.273248) (end 116.651752 96.904248) (width 0.3) (layer "F.Cu") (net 42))
 (segment (start 138.304752 102.454752) (end 139.167248 103.317248) (width 0.3) (layer "F.Cu") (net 42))
 (segment (start 150.443752 107.606248) (end 150.55 107.5) (width 0.3) (layer "F.Cu") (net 42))
 (segment (start 143.850732 103.317248) (end 148.139732 107.606248) (width 0.3) (layer "F.Cu") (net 42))
 (segment (start 116.651752 96.904248) (end 134.899512 96.904248) (width 0.3) (layer "F.Cu") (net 42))
 (segment (start 139.167248 103.317248) (end 143.850732 103.317248) (width 0.3) (layer "F.Cu") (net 42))
 (segment (start 134.899512 96.904248) (end 138.304752 100.309488) (width 0.3) (layer "F.Cu") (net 42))
 (via (at 150.55 107.5) (size 0.6) (drill 0.3) (layers "F.Cu" "B.Cu") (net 42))
 (segment (start 153.353248 110.303248) (end 157.490752 110.303248) (width 0.3) (layer "B.Cu") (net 42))
 (segment (start 150.55 107.5) (end 153.353248 110.303248) (width 0.3) (layer "B.Cu") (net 42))
 (segment (start 119.420752 95.753248) (end 120.809752 94.364248) (width 0.3) (layer "F.Cu") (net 23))
 (segment (start 120.809752 94.364248) (end 136.789752 94.364248) (width 0.3) (layer "F.Cu") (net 23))
 (segment (start 136.789752 94.364248) (end 139.420752 91.733248) (width 0.3) (layer "F.Cu") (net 23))
 (segment (start 120.571752 94.364248) (end 139.329752 94.364248) (width 0.3) (layer "B.Cu") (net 24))
 (segment (start 139.329752 94.364248) (end 139.420752 94.273248) (width 0.3) (layer "B.Cu") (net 24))
 (segment (start 119.420752 93.213248) (end 120.571752 94.364248) (width 0.3) (layer "B.Cu") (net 24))
 (segment (start 145.25 86.15) (end 145.416752 85.983248) (width 1) (layer "F.Cu") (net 1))
 (segment (start 162.05 108.284) (end 162.05 100.6) (width 1) (layer "F.Cu") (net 1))
 (segment (start 158.720752 86.373248) (end 154.044 91.05) (width 1) (layer "F.Cu") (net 1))
 (segment (start 154.044 91.05) (end 145.25 91.05) (width 1) (layer "F.Cu") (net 1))
 (segment (start 145.25 91.05) (end 145.25 86.15) (width 1) (layer "F.Cu") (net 1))
 (segment (start 145.416752 85.983248) (end 148.183252 85.983248) (width 1) (layer "F.Cu") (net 1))
 (segment (start 157.490752 112.843248) (end 162.05 108.284) (width 1) (layer "F.Cu") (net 1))
 (via (at 162.05 100.6) (size 0.8) (drill 0.3) (layers "F.Cu" "B.Cu") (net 1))
 (segment (start 138.443687 68.937248) (end 139.997817 68.937248) (width 1) (layer "B.Cu") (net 1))
 (segment (start 145.35 74.289431) (end 145.35 85.85) (width 1) (layer "B.Cu") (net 1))
 (segment (start 162.05 100.6) (end 158.720752 97.270752) (width 1) (layer "B.Cu") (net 1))
 (segment (start 119.420752 85.593248) (end 123.756752 85.593248) (width 1) (layer "B.Cu") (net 1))
 (segment (start 139.997817 68.937248) (end 145.35 74.289431) (width 1) (layer "B.Cu") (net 1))
 (segment (start 158.720752 97.270752) (end 158.720752 86.373248) (width 1) (layer "B.Cu") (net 1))
 (segment (start 137.3 70.080935) (end 138.443687 68.937248) (width 1) (layer "B.Cu") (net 1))
 (segment (start 145.483248 85.983248) (end 148.183252 85.983248) (width 1) (layer "B.Cu") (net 1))
 (segment (start 146.728252 87.438248) (end 148.183252 85.983248) (width 1) (layer "B.Cu") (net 1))
 (segment (start 116.95 86.6) (end 117.956752 85.593248) (width 1) (layer "B.Cu") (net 1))
 (segment (start 148.600752 98.873248) (end 146.728252 97.000748) (width 1) (layer "B.Cu") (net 1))
 (segment (start 146.728252 97.000748) (end 146.728252 87.438248) (width 1) (layer "B.Cu") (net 1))
 (segment (start 117.956752 85.593248) (end 119.420752 85.593248) (width 1) (layer "B.Cu") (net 1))
 (segment (start 114.020752 119.673248) (end 116.95 116.744) (width 1) (layer "B.Cu") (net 1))
 (segment (start 145.35 85.85) (end 145.483248 85.983248) (width 1) (layer "B.Cu") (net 1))
 (segment (start 116.95 116.744) (end 116.95 86.6) (width 1) (layer "B.Cu") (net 1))
 (segment (start 137.3 72.05) (end 137.3 70.080935) (width 1) (layer "B.Cu") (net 1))
 (segment (start 123.756752 85.593248) (end 137.3 72.05) (width 1) (layer "B.Cu") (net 1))
 (segment (start 139.420752 73.953248) (end 136.2 77.174) (width 1) (layer "F.Cu") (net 7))
 (segment (start 136.2 85.5) (end 136.106752 85.593248) (width 1) (layer "F.Cu") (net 7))
 (segment (start 158.720752 77.985748) (end 148.183252 88.523248) (width 1) (layer "F.Cu") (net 7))
 (segment (start 154.950752 107.763248) (end 148.600752 114.113248) (width 1) (layer "F.Cu") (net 7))
 (segment (start 136.106752 85.593248) (end 134.660752 85.593248) (width 1) (layer "F.Cu") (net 7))
 (segment (start 158.720752 76.373248) (end 152.223248 76.373248) (width 1) (layer "F.Cu") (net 7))
 (segment (start 148.183252 88.523248) (end 150.723248 88.523248) (width 1) (layer "F.Cu") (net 7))
 (segment (start 136.2 77.174) (end 136.2 85.5) (width 1) (layer "F.Cu") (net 7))
 (segment (start 139.746752 73.953248) (end 139.420752 73.953248) (width 1) (layer "F.Cu") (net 7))
 (segment (start 144.775 68.925) (end 139.746752 73.953248) (width 1) (layer "F.Cu") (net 7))
 (segment (start 158.720752 76.373248) (end 158.720752 77.985748) (width 1) (layer "F.Cu") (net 7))
 (segment (start 157.490752 107.763248) (end 154.950752 107.763248) (width 1) (layer "F.Cu") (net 7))
 (segment (start 150.080752 122.433248) (end 165.320752 122.433248) (width 1) (layer "F.Cu") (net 7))
 (segment (start 150.723248 88.523248) (end 150.95 88.75) (width 1) (layer "F.Cu") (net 7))
 (segment (start 152.223248 76.373248) (end 144.775 68.925) (width 1) (layer "F.Cu") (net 7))
 (via (at 150.95 88.75) (size 0.8) (drill 0.3) (layers "F.Cu" "B.Cu") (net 7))
 (segment (start 150.95 88.75) (end 157.490752 95.290752) (width 1) (layer "B.Cu") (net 7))
 (segment (start 157.490752 95.290752) (end 157.490752 107.763248) (width 1) (layer "B.Cu") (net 7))
 (segment (start 150.080752 122.433248) (end 150.080752 115.593248) (width 1) (layer "B.Cu") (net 7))
 (segment (start 150.080752 115.593248) (end 148.600752 114.113248) (width 1) (layer "B.Cu") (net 7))
 (segment (start 139.420752 86.653248) (end 142.630752 83.443248) (width 0.3) (layer "F.Cu") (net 21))
 (segment (start 142.630752 83.443248) (end 148.183252 83.443248) (width 0.3) (layer "F.Cu") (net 21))
 (segment (start 139.420752 79.033248) (end 141.290752 80.903248) (width 0.3) (layer "F.Cu") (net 18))
 (segment (start 141.290752 80.903248) (end 148.183252 80.903248) (width 0.3) (layer "F.Cu") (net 18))
 (segment (start 165.117752 95.476248) (end 169.020752 91.573248) (width 0.6) (layer "F.Cu") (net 8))
 (segment (start 156.562352 116.653248) (end 165.117752 108.097848) (width 0.6) (layer "F.Cu") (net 8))
 (segment (start 148.600752 116.653248) (end 156.562352 116.653248) (width 0.6) (layer "F.Cu") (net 8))
 (segment (start 165.117752 108.097848) (end 165.117752 95.476248) (width 0.6) (layer "F.Cu") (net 8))
 (segment (start 139.420752 101.893248) (end 141.480752 103.953248) (width 0.3) (layer "B.Cu") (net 3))
 (segment (start 141.480752 103.953248) (end 148.600752 103.953248) (width 0.3) (layer "B.Cu") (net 3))
 (segment (start 163.68 96.494) (end 148.600752 111.573248) (width 0.6) (layer "F.Cu") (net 6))
 (segment (start 169.488252 94.623248) (end 168.670752 94.623248) (width 0.2) (layer "F.Cu") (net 6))
 (segment (start 163.68 96.47) (end 163.68 96.494) (width 0.6) (layer "F.Cu") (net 6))
 (via (at 163.68 96.47) (size 1) (drill 0.3) (layers "F.Cu" "B.Cu") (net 6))
 (segment (start 163.68 96.47) (end 166.076752 94.073248) (width 0.6) (layer "B.Cu") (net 6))
 (segment (start 166.076752 94.073248) (end 169.020752 94.073248) (width 0.6) (layer "B.Cu") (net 6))
 (segment (start 148.600752 101.413248) (end 141.480752 101.413248) (width 0.3) (layer "B.Cu") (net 2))
 (segment (start 141.480752 101.413248) (end 139.420752 99.353248) (width 0.3) (layer "B.Cu") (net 2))
 (segment (start 119.420752 113.533248) (end 119.420752 119.520752) (width 0.3) (layer "F.Cu") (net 67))
 (segment (start 154.6 127.7) (end 155.160752 127.139248) (width 0.3) (layer "F.Cu") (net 67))
 (segment (start 119.420752 119.520752) (end 127.6 127.7) (width 0.3) (layer "F.Cu") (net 67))
 (segment (start 155.160752 127.139248) (end 155.160752 124.973248) (width 0.3) (layer "F.Cu") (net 67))
 (segment (start 127.6 127.7) (end 154.6 127.7) (width 0.3) (layer "F.Cu") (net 67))
 (segment (start 130.45 115.204) (end 130.45 122.2) (width 0.3) (layer "F.Cu") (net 65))
 (segment (start 134.660752 110.993248) (end 130.45 115.204) (width 0.3) (layer "F.Cu") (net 65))
 (via (at 130.45 122.2) (size 0.6) (drill 0.3) (layers "F.Cu" "B.Cu") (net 65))
 (segment (start 130.45 122.2) (end 136.772248 128.522248) (width 0.3) (layer "B.Cu") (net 65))
 (segment (start 136.772248 128.522248) (end 156.691752 128.522248) (width 0.3) (layer "B.Cu") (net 65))
 (segment (start 156.691752 128.522248) (end 160.240752 124.973248) (width 0.3) (layer "B.Cu") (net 65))
 (segment (start 128.423248 124.973248) (end 147.540752 124.973248) (width 0.3) (layer "F.Cu") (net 60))
 (segment (start 128 124.55) (end 128.423248 124.973248) (width 0.3) (layer "F.Cu") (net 60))
 (segment (start 128 107.45) (end 128 124.55) (width 0.3) (layer "F.Cu") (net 60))
 (via (at 128 107.45) (size 0.6) (drill 0.3) (layers "F.Cu" "B.Cu") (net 60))
 (segment (start 128 107.45) (end 127.95 107.4) (width 0.3) (layer "B.Cu") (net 60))
 (segment (start 127.95 107.4) (end 127.95 98.85) (width 0.3) (layer "B.Cu") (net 60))
 (segment (start 127.95 98.85) (end 128.506752 98.293248) (width 0.3) (layer "B.Cu") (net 60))
 (segment (start 128.506752 98.293248) (end 134.660752 98.293248) (width 0.3) (layer "B.Cu") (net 60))
 (segment (start 135.811752 110.370736) (end 135.811752 104.524248) (width 0.3) (layer "F.Cu") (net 62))
 (segment (start 156.361752 123.634248) (end 149.583281 123.634248) (width 0.3) (layer "F.Cu") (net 62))
 (segment (start 148.741752 121.232248) (end 140.678752 113.169248) (width 0.3) (layer "F.Cu") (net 62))
 (segment (start 138.610264 113.169248) (end 135.811752 110.370736) (width 0.3) (layer "F.Cu") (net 62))
 (segment (start 140.678752 113.169248) (end 138.610264 113.169248) (width 0.3) (layer "F.Cu") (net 62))
 (segment (start 135.811752 104.524248) (end 134.660752 103.373248) (width 0.3) (layer "F.Cu") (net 62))
 (segment (start 149.583281 123.634248) (end 148.741752 122.792719) (width 0.3) (layer "F.Cu") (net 62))
 (segment (start 157.700752 124.973248) (end 156.361752 123.634248) (width 0.3) (layer "F.Cu") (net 62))
 (segment (start 148.741752 122.792719) (end 148.741752 121.232248) (width 0.3) (layer "F.Cu") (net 62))
 (segment (start 132.520116 100.833248) (end 134.660752 100.833248) (width 0.3) (layer "F.Cu") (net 61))
 (segment (start 127.674248 126.174248) (end 126.35 124.85) (width 0.3) (layer "F.Cu") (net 61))
 (segment (start 126.35 124.85) (end 126.35 107.003363) (width 0.3) (layer "F.Cu") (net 61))
 (segment (start 126.35 107.003363) (end 132.520116 100.833248) (width 0.3) (layer "F.Cu") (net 61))
 (segment (start 150.080752 124.973248) (end 148.879752 126.174248) (width 0.3) (layer "F.Cu") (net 61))
 (segment (start 148.879752 126.174248) (end 127.674248 126.174248) (width 0.3) (layer "F.Cu") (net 61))
 (segment (start 129.2 122.6) (end 129.2 107.85) (width 0.3) (layer "F.Cu") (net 63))
 (segment (start 129.05 107.7) (end 130.836752 105.913248) (width 0.3) (layer "F.Cu") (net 63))
 (segment (start 130.836752 105.913248) (end 134.660752 105.913248) (width 0.3) (layer "F.Cu") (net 63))
 (segment (start 147.540752 122.433248) (end 145.634752 124.339248) (width 0.3) (layer "F.Cu") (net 63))
 (segment (start 129.2 107.85) (end 129.05 107.7) (width 0.3) (layer "F.Cu") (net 63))
 (segment (start 130.939248 124.339248) (end 129.2 122.6) (width 0.3) (layer "F.Cu") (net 63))
 (segment (start 145.634752 124.339248) (end 130.939248 124.339248) (width 0.3) (layer "F.Cu") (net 63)))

